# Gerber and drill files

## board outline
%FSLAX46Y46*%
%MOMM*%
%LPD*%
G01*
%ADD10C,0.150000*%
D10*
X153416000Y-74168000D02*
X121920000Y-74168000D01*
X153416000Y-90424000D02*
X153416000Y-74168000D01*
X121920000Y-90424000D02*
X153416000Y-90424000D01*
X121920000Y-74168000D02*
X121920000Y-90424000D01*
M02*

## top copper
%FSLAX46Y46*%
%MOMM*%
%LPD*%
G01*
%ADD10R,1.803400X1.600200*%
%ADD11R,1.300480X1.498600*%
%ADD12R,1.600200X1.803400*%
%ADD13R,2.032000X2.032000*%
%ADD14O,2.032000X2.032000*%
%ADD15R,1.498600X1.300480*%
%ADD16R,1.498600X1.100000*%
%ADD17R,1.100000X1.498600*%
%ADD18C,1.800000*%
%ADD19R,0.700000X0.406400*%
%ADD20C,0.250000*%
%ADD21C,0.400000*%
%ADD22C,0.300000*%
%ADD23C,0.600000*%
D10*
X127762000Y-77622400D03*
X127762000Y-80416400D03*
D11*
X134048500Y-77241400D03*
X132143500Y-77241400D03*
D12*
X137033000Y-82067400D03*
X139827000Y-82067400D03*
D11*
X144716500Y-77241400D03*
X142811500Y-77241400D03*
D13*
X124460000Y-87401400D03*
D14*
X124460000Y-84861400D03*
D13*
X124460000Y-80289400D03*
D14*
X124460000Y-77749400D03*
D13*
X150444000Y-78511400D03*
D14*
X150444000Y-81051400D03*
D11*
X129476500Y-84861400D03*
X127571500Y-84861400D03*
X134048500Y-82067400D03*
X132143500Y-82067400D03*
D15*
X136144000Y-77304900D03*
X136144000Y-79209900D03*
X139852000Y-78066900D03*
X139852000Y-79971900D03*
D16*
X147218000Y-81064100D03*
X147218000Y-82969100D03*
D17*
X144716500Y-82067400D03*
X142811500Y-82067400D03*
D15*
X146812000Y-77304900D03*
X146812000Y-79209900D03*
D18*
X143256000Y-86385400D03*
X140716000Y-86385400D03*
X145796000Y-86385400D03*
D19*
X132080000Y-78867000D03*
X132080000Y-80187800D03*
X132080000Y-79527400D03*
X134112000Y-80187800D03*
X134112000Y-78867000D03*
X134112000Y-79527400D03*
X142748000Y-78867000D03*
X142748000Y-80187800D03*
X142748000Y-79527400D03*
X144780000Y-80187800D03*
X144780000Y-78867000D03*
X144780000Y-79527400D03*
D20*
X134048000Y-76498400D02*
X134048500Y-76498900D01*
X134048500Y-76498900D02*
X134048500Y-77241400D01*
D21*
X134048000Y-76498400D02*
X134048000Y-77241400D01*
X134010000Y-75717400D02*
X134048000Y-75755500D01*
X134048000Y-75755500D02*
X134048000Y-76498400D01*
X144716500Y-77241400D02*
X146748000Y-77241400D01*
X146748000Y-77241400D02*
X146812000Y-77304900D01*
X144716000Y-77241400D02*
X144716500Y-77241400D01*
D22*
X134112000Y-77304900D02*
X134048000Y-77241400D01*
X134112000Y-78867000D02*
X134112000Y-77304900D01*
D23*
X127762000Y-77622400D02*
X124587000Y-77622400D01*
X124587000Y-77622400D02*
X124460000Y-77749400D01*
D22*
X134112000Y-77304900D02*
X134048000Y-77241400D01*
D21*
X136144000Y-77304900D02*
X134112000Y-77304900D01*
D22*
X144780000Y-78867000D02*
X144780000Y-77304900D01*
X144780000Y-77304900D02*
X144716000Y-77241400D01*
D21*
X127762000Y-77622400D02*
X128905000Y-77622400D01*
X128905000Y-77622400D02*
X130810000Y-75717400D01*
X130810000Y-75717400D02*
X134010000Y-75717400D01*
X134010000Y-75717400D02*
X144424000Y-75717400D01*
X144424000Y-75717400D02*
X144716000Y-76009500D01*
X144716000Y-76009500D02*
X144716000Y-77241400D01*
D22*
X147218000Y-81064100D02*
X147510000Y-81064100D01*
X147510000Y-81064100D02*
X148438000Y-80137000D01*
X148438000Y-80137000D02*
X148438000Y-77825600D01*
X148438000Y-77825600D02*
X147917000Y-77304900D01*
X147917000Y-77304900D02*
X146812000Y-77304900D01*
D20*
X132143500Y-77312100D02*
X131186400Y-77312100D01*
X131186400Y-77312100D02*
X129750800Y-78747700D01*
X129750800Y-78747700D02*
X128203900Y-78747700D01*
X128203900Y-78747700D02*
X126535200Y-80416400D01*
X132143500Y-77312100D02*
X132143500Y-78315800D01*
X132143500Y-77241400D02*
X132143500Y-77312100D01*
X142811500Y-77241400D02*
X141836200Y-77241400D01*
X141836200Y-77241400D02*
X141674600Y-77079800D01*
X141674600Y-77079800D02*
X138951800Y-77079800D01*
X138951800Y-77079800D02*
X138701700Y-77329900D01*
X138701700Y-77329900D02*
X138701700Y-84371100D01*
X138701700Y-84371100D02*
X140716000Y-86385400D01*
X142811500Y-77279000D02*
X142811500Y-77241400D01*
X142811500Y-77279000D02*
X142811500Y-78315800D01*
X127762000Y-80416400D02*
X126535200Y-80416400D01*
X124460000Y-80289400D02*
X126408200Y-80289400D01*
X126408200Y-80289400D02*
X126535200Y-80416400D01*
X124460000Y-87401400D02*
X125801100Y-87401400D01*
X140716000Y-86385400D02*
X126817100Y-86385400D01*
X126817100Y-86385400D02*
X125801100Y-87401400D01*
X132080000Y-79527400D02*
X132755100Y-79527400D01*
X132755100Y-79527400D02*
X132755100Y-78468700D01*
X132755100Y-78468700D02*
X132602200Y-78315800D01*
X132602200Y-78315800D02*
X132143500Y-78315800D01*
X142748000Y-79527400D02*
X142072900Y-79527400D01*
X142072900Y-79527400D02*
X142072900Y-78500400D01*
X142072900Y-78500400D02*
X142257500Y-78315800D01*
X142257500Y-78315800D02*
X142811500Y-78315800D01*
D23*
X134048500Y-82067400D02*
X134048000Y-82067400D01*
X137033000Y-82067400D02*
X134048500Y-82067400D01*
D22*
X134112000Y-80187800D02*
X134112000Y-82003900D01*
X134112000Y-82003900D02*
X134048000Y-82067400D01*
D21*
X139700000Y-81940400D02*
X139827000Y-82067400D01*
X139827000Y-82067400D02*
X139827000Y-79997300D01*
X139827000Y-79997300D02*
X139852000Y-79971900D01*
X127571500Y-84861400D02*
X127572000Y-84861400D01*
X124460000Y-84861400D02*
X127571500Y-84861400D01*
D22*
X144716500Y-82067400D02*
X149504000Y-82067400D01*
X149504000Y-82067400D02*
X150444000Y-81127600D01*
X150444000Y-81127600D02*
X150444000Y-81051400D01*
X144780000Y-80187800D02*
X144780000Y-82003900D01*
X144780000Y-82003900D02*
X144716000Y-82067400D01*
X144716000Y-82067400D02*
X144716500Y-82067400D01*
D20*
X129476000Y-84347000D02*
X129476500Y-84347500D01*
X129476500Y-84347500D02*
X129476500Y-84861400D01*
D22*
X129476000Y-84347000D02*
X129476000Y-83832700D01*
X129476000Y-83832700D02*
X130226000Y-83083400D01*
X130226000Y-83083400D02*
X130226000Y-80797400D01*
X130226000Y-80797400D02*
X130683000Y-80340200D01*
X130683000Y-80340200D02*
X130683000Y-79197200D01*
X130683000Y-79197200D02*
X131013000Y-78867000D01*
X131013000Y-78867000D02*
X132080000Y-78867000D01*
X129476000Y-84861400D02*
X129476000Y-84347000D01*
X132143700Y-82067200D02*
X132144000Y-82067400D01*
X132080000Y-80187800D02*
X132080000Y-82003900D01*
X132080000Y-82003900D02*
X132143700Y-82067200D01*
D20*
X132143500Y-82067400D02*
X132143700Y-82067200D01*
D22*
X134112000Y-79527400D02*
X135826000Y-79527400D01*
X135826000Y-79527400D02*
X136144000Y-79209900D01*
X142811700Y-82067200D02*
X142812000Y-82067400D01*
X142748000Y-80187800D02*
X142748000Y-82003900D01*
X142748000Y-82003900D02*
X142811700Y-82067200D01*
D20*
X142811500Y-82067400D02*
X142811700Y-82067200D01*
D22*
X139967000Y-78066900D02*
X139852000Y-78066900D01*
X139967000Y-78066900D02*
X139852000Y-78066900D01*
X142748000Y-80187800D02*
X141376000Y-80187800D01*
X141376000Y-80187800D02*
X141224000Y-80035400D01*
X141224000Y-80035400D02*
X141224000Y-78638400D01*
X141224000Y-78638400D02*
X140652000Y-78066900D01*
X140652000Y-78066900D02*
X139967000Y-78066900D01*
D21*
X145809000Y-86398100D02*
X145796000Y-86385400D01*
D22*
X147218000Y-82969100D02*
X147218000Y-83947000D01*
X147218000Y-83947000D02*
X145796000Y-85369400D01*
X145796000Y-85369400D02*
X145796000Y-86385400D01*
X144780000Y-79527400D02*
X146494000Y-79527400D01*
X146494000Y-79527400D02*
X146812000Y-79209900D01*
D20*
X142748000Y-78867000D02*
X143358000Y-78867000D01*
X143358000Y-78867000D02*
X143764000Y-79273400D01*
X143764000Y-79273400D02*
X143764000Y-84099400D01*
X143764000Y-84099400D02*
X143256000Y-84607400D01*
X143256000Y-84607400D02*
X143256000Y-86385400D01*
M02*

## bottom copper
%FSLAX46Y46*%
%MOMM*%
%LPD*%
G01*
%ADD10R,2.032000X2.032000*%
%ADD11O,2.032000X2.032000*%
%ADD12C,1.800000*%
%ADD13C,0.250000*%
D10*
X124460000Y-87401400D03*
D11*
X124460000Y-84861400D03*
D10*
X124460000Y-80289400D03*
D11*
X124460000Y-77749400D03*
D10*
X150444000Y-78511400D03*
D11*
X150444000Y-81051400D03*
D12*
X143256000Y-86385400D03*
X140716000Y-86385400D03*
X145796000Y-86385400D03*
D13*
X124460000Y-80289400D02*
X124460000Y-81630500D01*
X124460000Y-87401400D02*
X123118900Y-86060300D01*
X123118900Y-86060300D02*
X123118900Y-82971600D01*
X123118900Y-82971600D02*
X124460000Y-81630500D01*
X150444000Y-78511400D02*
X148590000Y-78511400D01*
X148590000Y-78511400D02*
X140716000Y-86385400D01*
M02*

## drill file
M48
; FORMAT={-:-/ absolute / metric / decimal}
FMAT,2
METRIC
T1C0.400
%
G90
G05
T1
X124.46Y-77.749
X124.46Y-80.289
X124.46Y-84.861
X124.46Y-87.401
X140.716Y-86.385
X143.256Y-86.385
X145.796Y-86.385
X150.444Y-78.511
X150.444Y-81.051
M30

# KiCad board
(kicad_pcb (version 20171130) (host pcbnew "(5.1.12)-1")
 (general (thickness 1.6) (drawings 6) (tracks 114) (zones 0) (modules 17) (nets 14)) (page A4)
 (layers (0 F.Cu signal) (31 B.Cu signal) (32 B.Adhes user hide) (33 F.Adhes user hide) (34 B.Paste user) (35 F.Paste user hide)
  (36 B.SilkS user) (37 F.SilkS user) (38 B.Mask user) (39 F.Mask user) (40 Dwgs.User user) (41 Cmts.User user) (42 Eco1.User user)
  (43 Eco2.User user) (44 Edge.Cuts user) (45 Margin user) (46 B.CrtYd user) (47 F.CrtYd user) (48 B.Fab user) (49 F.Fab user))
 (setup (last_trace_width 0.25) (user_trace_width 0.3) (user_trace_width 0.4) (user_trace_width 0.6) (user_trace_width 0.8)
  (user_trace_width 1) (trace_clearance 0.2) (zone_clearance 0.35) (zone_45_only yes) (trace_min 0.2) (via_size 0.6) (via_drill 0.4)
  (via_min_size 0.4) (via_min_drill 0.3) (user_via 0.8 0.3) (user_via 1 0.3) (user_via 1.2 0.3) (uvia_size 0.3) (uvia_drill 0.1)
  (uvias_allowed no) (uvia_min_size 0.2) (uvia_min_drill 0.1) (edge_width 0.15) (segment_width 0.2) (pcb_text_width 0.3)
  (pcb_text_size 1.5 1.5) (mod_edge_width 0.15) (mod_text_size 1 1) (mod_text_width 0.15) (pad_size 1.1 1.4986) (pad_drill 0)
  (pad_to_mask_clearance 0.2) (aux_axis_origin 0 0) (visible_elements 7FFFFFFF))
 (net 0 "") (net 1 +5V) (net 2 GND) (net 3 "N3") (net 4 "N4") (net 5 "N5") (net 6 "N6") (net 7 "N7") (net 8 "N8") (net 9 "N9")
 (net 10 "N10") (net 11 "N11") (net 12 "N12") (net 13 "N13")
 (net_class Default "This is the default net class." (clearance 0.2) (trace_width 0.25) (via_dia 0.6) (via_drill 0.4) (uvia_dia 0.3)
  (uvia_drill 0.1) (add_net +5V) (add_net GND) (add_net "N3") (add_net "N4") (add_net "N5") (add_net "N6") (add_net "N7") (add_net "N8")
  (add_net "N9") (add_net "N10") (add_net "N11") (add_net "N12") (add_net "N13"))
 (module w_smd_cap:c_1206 (layer F.Cu) (at 127.762 79.0194 90)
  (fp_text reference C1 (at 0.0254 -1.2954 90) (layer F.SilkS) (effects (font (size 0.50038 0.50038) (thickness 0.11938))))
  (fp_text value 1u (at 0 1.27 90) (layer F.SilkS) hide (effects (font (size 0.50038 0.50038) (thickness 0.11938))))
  (pad 1 smd rect (at 1.397 0 90) (size 1.6002 1.8034) (layers F.Cu F.Paste F.Mask) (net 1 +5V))
  (pad 2 smd rect (at -1.397 0 90) (size 1.6002 1.8034) (layers F.Cu F.Paste F.Mask) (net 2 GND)))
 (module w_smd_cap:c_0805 (layer F.Cu) (at 133.096 77.2414)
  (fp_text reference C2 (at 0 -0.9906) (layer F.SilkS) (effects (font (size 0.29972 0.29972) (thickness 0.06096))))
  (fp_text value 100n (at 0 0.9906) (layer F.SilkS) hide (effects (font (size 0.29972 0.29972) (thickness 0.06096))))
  (pad 1 smd rect (at 0.9525 0) (size 1.30048 1.4986) (layers F.Cu F.Paste F.Mask) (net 1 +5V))
  (pad 2 smd rect (at -0.9525 0) (size 1.30048 1.4986) (layers F.Cu F.Paste F.Mask) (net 2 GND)))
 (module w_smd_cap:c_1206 (layer F.Cu) (at 138.43 82.0674 180)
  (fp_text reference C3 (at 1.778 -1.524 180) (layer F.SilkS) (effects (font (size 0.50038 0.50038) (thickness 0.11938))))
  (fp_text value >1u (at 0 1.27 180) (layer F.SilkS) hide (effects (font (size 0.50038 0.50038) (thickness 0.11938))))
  (pad 1 smd rect (at 1.397 0 180) (size 1.6002 1.8034) (layers F.Cu F.Paste F.Mask) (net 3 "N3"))
  (pad 2 smd rect (at -1.397 0 180) (size 1.6002 1.8034) (layers F.Cu F.Paste F.Mask) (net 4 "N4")))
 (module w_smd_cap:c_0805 (layer F.Cu) (at 143.764 77.2414)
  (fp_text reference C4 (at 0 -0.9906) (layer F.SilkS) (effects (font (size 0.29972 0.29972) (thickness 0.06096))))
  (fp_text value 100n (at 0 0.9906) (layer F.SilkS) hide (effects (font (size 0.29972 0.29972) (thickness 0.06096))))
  (pad 1 smd rect (at 0.9525 0) (size 1.30048 1.4986) (layers F.Cu F.Paste F.Mask) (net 1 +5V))
  (pad 2 smd rect (at -0.9525 0) (size 1.30048 1.4986) (layers F.Cu F.Paste F.Mask) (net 2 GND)))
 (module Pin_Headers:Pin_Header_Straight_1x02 (layer F.Cu) (at 124.46 87.4014 180)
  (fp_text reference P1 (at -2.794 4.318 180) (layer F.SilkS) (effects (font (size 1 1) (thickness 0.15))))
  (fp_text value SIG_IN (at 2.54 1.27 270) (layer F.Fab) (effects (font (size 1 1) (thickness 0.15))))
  (pad 1 thru_hole rect (at 0 0 180) (size 2.032 2.032) (drill 0.4) (layers *.Cu *.Mask F.SilkS) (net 2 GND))
  (pad 2 thru_hole oval (at 0 2.54 180) (size 2.032 2.032) (drill 0.4) (layers *.Cu *.Mask F.SilkS) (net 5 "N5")))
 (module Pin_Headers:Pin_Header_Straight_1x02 (layer F.Cu) (at 124.46 80.2894 180)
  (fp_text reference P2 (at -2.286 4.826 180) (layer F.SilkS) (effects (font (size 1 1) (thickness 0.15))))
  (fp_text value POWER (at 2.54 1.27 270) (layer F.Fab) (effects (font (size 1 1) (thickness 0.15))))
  (pad 1 thru_hole rect (at 0 0 180) (size 2.032 2.032) (drill 0.4) (layers *.Cu *.Mask F.SilkS) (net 2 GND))
  (pad 2 thru_hole oval (at 0 2.54 180) (size 2.032 2.032) (drill 0.4) (layers *.Cu *.Mask F.SilkS) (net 1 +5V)))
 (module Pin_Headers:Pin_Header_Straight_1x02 (layer F.Cu) (at 150.444 78.5114)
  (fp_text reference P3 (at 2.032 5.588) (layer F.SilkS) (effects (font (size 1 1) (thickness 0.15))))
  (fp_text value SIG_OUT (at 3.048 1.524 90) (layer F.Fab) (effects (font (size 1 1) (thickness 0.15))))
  (pad 1 thru_hole rect (at 0 0) (size 2.032 2.032) (drill 0.4) (layers *.Cu *.Mask F.SilkS) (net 2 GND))
  (pad 2 thru_hole oval (at 0 2.54) (size 2.032 2.032) (drill 0.4) (layers *.Cu *.Mask F.SilkS) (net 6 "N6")))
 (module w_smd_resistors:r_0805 (layer F.Cu) (at 128.524 84.8614)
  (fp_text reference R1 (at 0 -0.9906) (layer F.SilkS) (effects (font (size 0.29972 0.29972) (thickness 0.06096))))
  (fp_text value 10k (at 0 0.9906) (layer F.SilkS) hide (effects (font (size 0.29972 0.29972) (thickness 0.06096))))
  (pad 1 smd rect (at 0.9525 0) (size 1.30048 1.4986) (layers F.Cu F.Paste F.Mask) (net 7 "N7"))
  (pad 2 smd rect (at -0.9525 0) (size 1.30048 1.4986) (layers F.Cu F.Paste F.Mask) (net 5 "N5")))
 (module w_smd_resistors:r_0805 (layer F.Cu) (at 133.096 82.0674)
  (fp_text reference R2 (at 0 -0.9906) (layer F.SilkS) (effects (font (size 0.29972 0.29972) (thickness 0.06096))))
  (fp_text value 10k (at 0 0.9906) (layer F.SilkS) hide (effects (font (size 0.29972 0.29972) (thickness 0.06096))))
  (pad 1 smd rect (at 0.9525 0) (size 1.30048 1.4986) (layers F.Cu F.Paste F.Mask) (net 3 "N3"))
  (pad 2 smd rect (at -0.9525 0) (size 1.30048 1.4986) (layers F.Cu F.Paste F.Mask) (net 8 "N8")))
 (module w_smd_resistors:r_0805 (layer F.Cu) (at 136.144 78.2574 90)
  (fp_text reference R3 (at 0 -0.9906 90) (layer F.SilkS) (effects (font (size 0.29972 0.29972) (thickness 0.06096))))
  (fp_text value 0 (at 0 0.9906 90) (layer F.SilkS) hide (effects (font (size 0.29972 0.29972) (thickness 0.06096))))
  (pad 1 smd rect (at 0.9525 0 90) (size 1.30048 1.4986) (layers F.Cu F.Paste F.Mask) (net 1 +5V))
  (pad 2 smd rect (at -0.9525 0 90) (size 1.30048 1.4986) (layers F.Cu F.Paste F.Mask) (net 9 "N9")))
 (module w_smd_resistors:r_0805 (layer F.Cu) (at 139.852 79.0194 90)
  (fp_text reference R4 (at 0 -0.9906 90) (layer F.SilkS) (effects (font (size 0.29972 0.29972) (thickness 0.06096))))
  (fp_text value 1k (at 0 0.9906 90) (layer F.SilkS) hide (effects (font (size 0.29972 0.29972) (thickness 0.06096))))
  (pad 1 smd rect (at 0.9525 0 90) (size 1.30048 1.4986) (layers F.Cu F.Paste F.Mask) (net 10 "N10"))
  (pad 2 smd rect (at -0.9525 0 90) (size 1.30048 1.4986) (layers F.Cu F.Paste F.Mask) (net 4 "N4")))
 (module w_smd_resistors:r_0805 (layer F.Cu) (at 147.218 82.0166 90)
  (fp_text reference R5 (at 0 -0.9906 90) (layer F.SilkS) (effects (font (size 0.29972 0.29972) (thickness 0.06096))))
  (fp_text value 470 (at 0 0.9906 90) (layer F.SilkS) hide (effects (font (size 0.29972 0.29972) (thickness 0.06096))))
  (pad 1 smd rect (at 0.9525 0 90) (size 1.1 1.4986) (layers F.Cu F.Paste F.Mask) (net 1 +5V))
  (pad 2 smd rect (at -0.9525 0 90) (size 1.1 1.4986) (layers F.Cu F.Paste F.Mask) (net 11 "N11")))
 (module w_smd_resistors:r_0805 (layer F.Cu) (at 143.764 82.0674)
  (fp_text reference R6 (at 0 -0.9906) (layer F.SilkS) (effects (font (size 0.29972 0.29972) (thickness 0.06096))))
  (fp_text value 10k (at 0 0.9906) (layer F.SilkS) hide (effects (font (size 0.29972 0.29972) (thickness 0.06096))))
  (pad 1 smd rect (at 0.9525 0) (size 1.1 1.4986) (layers F.Cu F.Paste F.Mask) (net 6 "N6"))
  (pad 2 smd rect (at -0.9525 0) (size 1.1 1.4986) (layers F.Cu F.Paste F.Mask) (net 10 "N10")))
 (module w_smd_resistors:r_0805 (layer F.Cu) (at 146.812 78.2574 90)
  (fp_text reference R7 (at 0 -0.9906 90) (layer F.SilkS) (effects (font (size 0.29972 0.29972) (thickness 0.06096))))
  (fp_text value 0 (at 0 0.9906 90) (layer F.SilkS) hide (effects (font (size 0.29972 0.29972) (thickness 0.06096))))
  (pad 1 smd rect (at 0.9525 0 90) (size 1.30048 1.4986) (layers F.Cu F.Paste F.Mask) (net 1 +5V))
  (pad 2 smd rect (at -0.9525 0 90) (size 1.30048 1.4986) (layers F.Cu F.Paste F.Mask) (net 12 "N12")))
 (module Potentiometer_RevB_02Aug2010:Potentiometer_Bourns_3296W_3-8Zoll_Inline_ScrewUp (layer F.Cu) (at 143.256 86.3854 90)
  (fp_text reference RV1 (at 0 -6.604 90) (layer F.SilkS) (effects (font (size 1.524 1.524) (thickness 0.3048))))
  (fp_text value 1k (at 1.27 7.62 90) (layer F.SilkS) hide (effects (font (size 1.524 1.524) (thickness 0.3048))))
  (pad 2 thru_hole circle (at 0 0 90) (size 1.8 1.8) (drill 0.4) (layers *.Cu *.Mask F.SilkS) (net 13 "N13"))
  (pad 3 thru_hole circle (at 0 -2.54 90) (size 1.8 1.8) (drill 0.4) (layers *.Cu *.Mask F.SilkS) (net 2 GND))
  (pad 1 thru_hole circle (at 0 2.54 90) (size 1.8 1.8) (drill 0.4) (layers *.Cu *.Mask F.SilkS) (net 11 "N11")))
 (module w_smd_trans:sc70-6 (layer F.Cu) (at 133.096 79.5274 270)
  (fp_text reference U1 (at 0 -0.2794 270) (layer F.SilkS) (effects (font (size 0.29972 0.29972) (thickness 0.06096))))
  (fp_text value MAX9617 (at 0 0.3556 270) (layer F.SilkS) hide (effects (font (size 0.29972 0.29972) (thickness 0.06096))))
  (pad 1 smd rect (at -0.6604 1.016 270) (size 0.4064 0.7) (layers F.Cu F.Paste F.Mask) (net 7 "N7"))
  (pad 3 smd rect (at 0.6604 1.016 270) (size 0.4064 0.7) (layers F.Cu F.Paste F.Mask) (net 8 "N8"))
  (pad 2 smd rect (at 0 1.016 270) (size 0.4064 0.7) (layers F.Cu F.Paste F.Mask) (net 2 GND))
  (pad 4 smd rect (at 0.6604 -1.016 270) (size 0.4064 0.7) (layers F.Cu F.Paste F.Mask) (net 3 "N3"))
  (pad 6 smd rect (at -0.6604 -1.016 270) (size 0.4064 0.7) (layers F.Cu F.Paste F.Mask) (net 1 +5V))
  (pad 5 smd rect (at 0 -1.016 270) (size 0.4064 0.7) (layers F.Cu F.Paste F.Mask) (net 9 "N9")))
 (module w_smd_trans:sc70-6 (layer F.Cu) (at 143.764 79.5274 270)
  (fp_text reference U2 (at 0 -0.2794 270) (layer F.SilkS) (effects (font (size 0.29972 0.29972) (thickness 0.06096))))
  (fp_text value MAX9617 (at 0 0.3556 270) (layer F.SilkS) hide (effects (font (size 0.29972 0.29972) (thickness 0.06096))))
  (pad 1 smd rect (at -0.6604 1.016 270) (size 0.4064 0.7) (layers F.Cu F.Paste F.Mask) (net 13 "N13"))
  (pad 3 smd rect (at 0.6604 1.016 270) (size 0.4064 0.7) (layers F.Cu F.Paste F.Mask) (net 10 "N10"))
  (pad 2 smd rect (at 0 1.016 270) (size 0.4064 0.7) (layers F.Cu F.Paste F.Mask) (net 2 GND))
  (pad 4 smd rect (at 0.6604 -1.016 270) (size 0.4064 0.7) (layers F.Cu F.Paste F.Mask) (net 6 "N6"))
  (pad 6 smd rect (at -0.6604 -1.016 270) (size 0.4064 0.7) (layers F.Cu F.Paste F.Mask) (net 1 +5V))
  (pad 5 smd rect (at 0 -1.016 270) (size 0.4064 0.7) (layers F.Cu F.Paste F.Mask) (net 12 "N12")))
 (gr_line (start 153.416 74.168) (end 121.92 74.168) (angle 90) (layer Edge.Cuts) (width 0.15))
 (gr_line (start 153.416 90.424) (end 153.416 74.168) (angle 90) (layer Edge.Cuts) (width 0.15))
 (gr_line (start 121.92 90.424) (end 153.416 90.424) (angle 90) (layer Edge.Cuts) (width 0.15))
 (gr_line (start 121.92 74.168) (end 121.92 90.424) (angle 90) (layer Edge.Cuts) (width 0.15))
 (segment (start 134.048 76.4984) (end 134.0485 76.4989) (width 0.25) (layer F.Cu) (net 1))
 (segment (start 134.0485 76.4989) (end 134.0485 77.2414) (width 0.25) (layer F.Cu) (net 1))
 (segment (start 134.048 76.4984) (end 134.048 77.2414) (width 0.4) (layer F.Cu) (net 1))
 (segment (start 134.01 75.7174) (end 134.048 75.7555) (width 0.4) (layer F.Cu) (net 1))
 (segment (start 134.048 75.7555) (end 134.048 76.4984) (width 0.4) (layer F.Cu) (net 1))
 (segment (start 144.7165 77.2414) (end 146.748 77.2414) (width 0.4) (layer F.Cu) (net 1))
 (segment (start 146.748 77.2414) (end 146.812 77.3049) (width 0.4) (layer F.Cu) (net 1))
 (segment (start 144.716 77.2414) (end 144.7165 77.2414) (width 0.4) (layer F.Cu) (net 1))
 (segment (start 134.112 77.3049) (end 134.048 77.2414) (width 0.3) (layer F.Cu) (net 1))
 (segment (start 134.112 78.867) (end 134.112 77.3049) (width 0.3) (layer F.Cu) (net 1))
 (segment (start 127.762 77.6224) (end 124.587 77.6224) (width 0.6) (layer F.Cu) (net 1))
 (segment (start 124.587 77.6224) (end 124.46 77.7494) (width 0.6) (layer F.Cu) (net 1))
 (segment (start 134.112 77.3049) (end 134.048 77.2414) (width 0.3) (layer F.Cu) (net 1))
 (segment (start 136.144 77.3049) (end 134.112 77.3049) (width 0.4) (layer F.Cu) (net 1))
 (segment (start 144.78 78.867) (end 144.78 77.3049) (width 0.3) (layer F.Cu) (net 1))
 (segment (start 144.78 77.3049) (end 144.716 77.2414) (width 0.3) (layer F.Cu) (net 1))
 (segment (start 127.762 77.6224) (end 128.905 77.6224) (width 0.4) (layer F.Cu) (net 1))
 (segment (start 128.905 77.6224) (end 130.81 75.7174) (width 0.4) (layer F.Cu) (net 1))
 (segment (start 130.81 75.7174) (end 134.01 75.7174) (width 0.4) (layer F.Cu) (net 1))
 (segment (start 134.01 75.7174) (end 144.424 75.7174) (width 0.4) (layer F.Cu) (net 1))
 (segment (start 144.424 75.7174) (end 144.716 76.0095) (width 0.4) (layer F.Cu) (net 1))
 (segment (start 144.716 76.0095) (end 144.716 77.2414) (width 0.4) (layer F.Cu) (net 1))
 (segment (start 147.218 81.0641) (end 147.51 81.0641) (width 0.3) (layer F.Cu) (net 1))
 (segment (start 147.51 81.0641) (end 148.438 80.137) (width 0.3) (layer F.Cu) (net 1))
 (segment (start 148.438 80.137) (end 148.438 77.8256) (width 0.3) (layer F.Cu) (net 1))
 (segment (start 148.438 77.8256) (end 147.917 77.3049) (width 0.3) (layer F.Cu) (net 1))
 (segment (start 147.917 77.3049) (end 146.812 77.3049) (width 0.3) (layer F.Cu) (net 1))
 (segment (start 132.1435 77.3121) (end 131.1864 77.3121) (width 0.25) (layer F.Cu) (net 2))
 (segment (start 131.1864 77.3121) (end 129.7508 78.7477) (width 0.25) (layer F.Cu) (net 2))
 (segment (start 129.7508 78.7477) (end 128.2039 78.7477) (width 0.25) (layer F.Cu) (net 2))
 (segment (start 128.2039 78.7477) (end 126.5352 80.4164) (width 0.25) (layer F.Cu) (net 2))
 (segment (start 132.1435 77.3121) (end 132.1435 78.3158) (width 0.25) (layer F.Cu) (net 2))
 (segment (start 132.1435 77.2414) (end 132.1435 77.3121) (width 0.25) (layer F.Cu) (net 2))
 (segment (start 142.8115 77.2414) (end 141.8362 77.2414) (width 0.25) (layer F.Cu) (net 2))
 (segment (start 141.8362 77.2414) (end 141.6746 77.0798) (width 0.25) (layer F.Cu) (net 2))
 (segment (start 141.6746 77.0798) (end 138.9518 77.0798) (width 0.25) (layer F.Cu) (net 2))
 (segment (start 138.9518 77.0798) (end 138.7017 77.3299) (width 0.25) (layer F.Cu) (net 2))
 (segment (start 138.7017 77.3299) (end 138.7017 84.3711) (width 0.25) (layer F.Cu) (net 2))
 (segment (start 138.7017 84.3711) (end 140.716 86.3854) (width 0.25) (layer F.Cu) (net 2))
 (segment (start 142.8115 77.279) (end 142.8115 77.2414) (width 0.25) (layer F.Cu) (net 2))
 (segment (start 142.8115 77.279) (end 142.8115 78.3158) (width 0.25) (layer F.Cu) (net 2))
 (segment (start 124.46 80.2894) (end 124.46 81.6305) (width 0.25) (layer B.Cu) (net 2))
 (segment (start 124.46 87.4014) (end 123.1189 86.0603) (width 0.25) (layer B.Cu) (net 2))
 (segment (start 123.1189 86.0603) (end 123.1189 82.9716) (width 0.25) (layer B.Cu) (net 2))
 (segment (start 123.1189 82.9716) (end 124.46 81.6305) (width 0.25) (layer B.Cu) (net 2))
 (segment (start 127.762 80.4164) (end 126.5352 80.4164) (width 0.25) (layer F.Cu) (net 2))
 (segment (start 124.46 80.2894) (end 126.4082 80.2894) (width 0.25) (layer F.Cu) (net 2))
 (segment (start 126.4082 80.2894) (end 126.5352 80.4164) (width 0.25) (layer F.Cu) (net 2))
 (segment (start 150.444 78.5114) (end 148.59 78.5114) (width 0.25) (layer B.Cu) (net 2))
 (segment (start 148.59 78.5114) (end 140.716 86.3854) (width 0.25) (layer B.Cu) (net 2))
 (segment (start 124.46 87.4014) (end 125.8011 87.4014) (width 0.25) (layer F.Cu) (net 2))
 (segment (start 140.716 86.3854) (end 126.8171 86.3854) (width 0.25) (layer F.Cu) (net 2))
 (segment (start 126.8171 86.3854) (end 125.8011 87.4014) (width 0.25) (layer F.Cu) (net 2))
 (segment (start 132.08 79.5274) (end 132.7551 79.5274) (width 0.25) (layer F.Cu) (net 2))
 (segment (start 132.7551 79.5274) (end 132.7551 78.4687) (width 0.25) (layer F.Cu) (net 2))
 (segment (start 132.7551 78.4687) (end 132.6022 78.3158) (width 0.25) (layer F.Cu) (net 2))
 (segment (start 132.6022 78.3158) (end 132.1435 78.3158) (width 0.25) (layer F.Cu) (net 2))
 (segment (start 142.748 79.5274) (end 142.0729 79.5274) (width 0.25) (layer F.Cu) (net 2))
 (segment (start 142.0729 79.5274) (end 142.0729 78.5004) (width 0.25) (layer F.Cu) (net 2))
 (segment (start 142.0729 78.5004) (end 142.2575 78.3158) (width 0.25) (layer F.Cu) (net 2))
 (segment (start 142.2575 78.3158) (end 142.8115 78.3158) (width 0.25) (layer F.Cu) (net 2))
 (segment (start 134.0485 82.0674) (end 134.048 82.0674) (width 0.6) (layer F.Cu) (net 3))
 (segment (start 137.033 82.0674) (end 134.0485 82.0674) (width 0.6) (layer F.Cu) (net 3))
 (segment (start 134.112 80.1878) (end 134.112 82.0039) (width 0.3) (layer F.Cu) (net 3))
 (segment (start 134.112 82.0039) (end 134.048 82.0674) (width 0.3) (layer F.Cu) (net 3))
 (segment (start 139.7 81.9404) (end 139.827 82.0674) (width 0.4) (layer F.Cu) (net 4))
 (segment (start 139.827 82.0674) (end 139.827 79.9973) (width 0.4) (layer F.Cu) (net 4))
 (segment (start 139.827 79.9973) (end 139.852 79.9719) (width 0.4) (layer F.Cu) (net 4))
 (segment (start 127.5715 84.8614) (end 127.572 84.8614) (width 0.4) (layer F.Cu) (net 5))
 (segment (start 124.46 84.8614) (end 127.5715 84.8614) (width 0.4) (layer F.Cu) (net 5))
 (segment (start 144.7165 82.0674) (end 149.504 82.0674) (width 0.3) (layer F.Cu) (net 6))
 (segment (start 149.504 82.0674) (end 150.444 81.1276) (width 0.3) (layer F.Cu) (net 6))
 (segment (start 150.444 81.1276) (end 150.444 81.0514) (width 0.3) (layer F.Cu) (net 6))
 (segment (start 144.78 80.1878) (end 144.78 82.0039) (width 0.3) (layer F.Cu) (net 6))
 (segment (start 144.78 82.0039) (end 144.716 82.0674) (width 0.3) (layer F.Cu) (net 6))
 (segment (start 144.716 82.0674) (end 144.7165 82.0674) (width 0.3) (layer F.Cu) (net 6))
 (segment (start 129.476 84.347) (end 129.4765 84.3475) (width 0.25) (layer F.Cu) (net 7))
 (segment (start 129.4765 84.3475) (end 129.4765 84.8614) (width 0.25) (layer F.Cu) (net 7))
 (segment (start 129.476 84.347) (end 129.476 83.8327) (width 0.3) (layer F.Cu) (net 7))
 (segment (start 129.476 83.8327) (end 130.226 83.0834) (width 0.3) (layer F.Cu) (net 7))
 (segment (start 130.226 83.0834) (end 130.226 80.7974) (width 0.3) (layer F.Cu) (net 7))
 (segment (start 130.226 80.7974) (end 130.683 80.3402) (width 0.3) (layer F.Cu) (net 7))
 (segment (start 130.683 80.3402) (end 130.683 79.1972) (width 0.3) (layer F.Cu) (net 7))
 (segment (start 130.683 79.1972) (end 131.013 78.867) (width 0.3) (layer F.Cu) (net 7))
 (segment (start 131.013 78.867) (end 132.08 78.867) (width 0.3) (layer F.Cu) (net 7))
 (segment (start 129.476 84.8614) (end 129.476 84.347) (width 0.3) (layer F.Cu) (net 7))
 (segment (start 132.1437 82.0672) (end 132.144 82.0674) (width 0.3) (layer F.Cu) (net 8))
 (segment (start 132.08 80.1878) (end 132.08 82.0039) (width 0.3) (layer F.Cu) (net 8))
 (segment (start 132.08 82.0039) (end 132.1437 82.0672) (width 0.3) (layer F.Cu) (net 8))
 (segment (start 132.1435 82.0674) (end 132.1437 82.0672) (width 0.25) (layer F.Cu) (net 8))
 (segment (start 134.112 79.5274) (end 135.826 79.5274) (width 0.3) (layer F.Cu) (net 9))
 (segment (start 135.826 79.5274) (end 136.144 79.2099) (width 0.3) (layer F.Cu) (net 9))
 (segment (start 142.8117 82.0672) (end 142.812 82.0674) (width 0.3) (layer F.Cu) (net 10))
 (segment (start 142.748 80.1878) (end 142.748 82.0039) (width 0.3) (layer F.Cu) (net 10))
 (segment (start 142.748 82.0039) (end 142.8117 82.0672) (width 0.3) (layer F.Cu) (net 10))
 (segment (start 142.8115 82.0674) (end 142.8117 82.0672) (width 0.25) (layer F.Cu) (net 10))
 (segment (start 139.967 78.0669) (end 139.852 78.0669) (width 0.3) (layer F.Cu) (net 10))
 (segment (start 139.967 78.0669) (end 139.852 78.0669) (width 0.3) (layer F.Cu) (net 10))
 (segment (start 142.748 80.1878) (end 141.376 80.1878) (width 0.3) (layer F.Cu) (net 10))
 (segment (start 141.376 80.1878) (end 141.224 80.0354) (width 0.3) (layer F.Cu) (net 10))
 (segment (start 141.224 80.0354) (end 141.224 78.6384) (width 0.3) (layer F.Cu) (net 10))
 (segment (start 141.224 78.6384) (end 140.652 78.0669) (width 0.3) (layer F.Cu) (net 10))
 (segment (start 140.652 78.0669) (end 139.967 78.0669) (width 0.3) (layer F.Cu) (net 10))
 (segment (start 145.809 86.3981) (end 145.796 86.3854) (width 0.4) (layer F.Cu) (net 11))
 (segment (start 147.218 82.9691) (end 147.218 83.947) (width 0.3) (layer F.Cu) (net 11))
 (segment (start 147.218 83.947) (end 145.796 85.3694) (width 0.3) (layer F.Cu) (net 11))
 (segment (start 145.796 85.3694) (end 145.796 86.3854) (width 0.3) (layer F.Cu) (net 11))
 (segment (start 144.78 79.5274) (end 146.494 79.5274) (width 0.3) (layer F.Cu) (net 12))
 (segment (start 146.494 79.5274) (end 146.812 79.2099) (width 0.3) (layer F.Cu) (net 12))
 (segment (start 142.748 78.867) (end 143.358 78.867) (width 0.25) (layer F.Cu) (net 13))
 (segment (start 143.358 78.867) (end 143.764 79.2734) (width 0.25) (layer F.Cu) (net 13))
 (segment (start 143.764 79.2734) (end 143.764 84.0994) (width 0.25) (layer F.Cu) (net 13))
 (segment (start 143.764 84.0994) (end 143.256 84.6074) (width 0.25) (layer F.Cu) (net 13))
 (segment (start 143.256 84.6074) (end 143.256 86.3854) (width 0.25) (layer F.Cu) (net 13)))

